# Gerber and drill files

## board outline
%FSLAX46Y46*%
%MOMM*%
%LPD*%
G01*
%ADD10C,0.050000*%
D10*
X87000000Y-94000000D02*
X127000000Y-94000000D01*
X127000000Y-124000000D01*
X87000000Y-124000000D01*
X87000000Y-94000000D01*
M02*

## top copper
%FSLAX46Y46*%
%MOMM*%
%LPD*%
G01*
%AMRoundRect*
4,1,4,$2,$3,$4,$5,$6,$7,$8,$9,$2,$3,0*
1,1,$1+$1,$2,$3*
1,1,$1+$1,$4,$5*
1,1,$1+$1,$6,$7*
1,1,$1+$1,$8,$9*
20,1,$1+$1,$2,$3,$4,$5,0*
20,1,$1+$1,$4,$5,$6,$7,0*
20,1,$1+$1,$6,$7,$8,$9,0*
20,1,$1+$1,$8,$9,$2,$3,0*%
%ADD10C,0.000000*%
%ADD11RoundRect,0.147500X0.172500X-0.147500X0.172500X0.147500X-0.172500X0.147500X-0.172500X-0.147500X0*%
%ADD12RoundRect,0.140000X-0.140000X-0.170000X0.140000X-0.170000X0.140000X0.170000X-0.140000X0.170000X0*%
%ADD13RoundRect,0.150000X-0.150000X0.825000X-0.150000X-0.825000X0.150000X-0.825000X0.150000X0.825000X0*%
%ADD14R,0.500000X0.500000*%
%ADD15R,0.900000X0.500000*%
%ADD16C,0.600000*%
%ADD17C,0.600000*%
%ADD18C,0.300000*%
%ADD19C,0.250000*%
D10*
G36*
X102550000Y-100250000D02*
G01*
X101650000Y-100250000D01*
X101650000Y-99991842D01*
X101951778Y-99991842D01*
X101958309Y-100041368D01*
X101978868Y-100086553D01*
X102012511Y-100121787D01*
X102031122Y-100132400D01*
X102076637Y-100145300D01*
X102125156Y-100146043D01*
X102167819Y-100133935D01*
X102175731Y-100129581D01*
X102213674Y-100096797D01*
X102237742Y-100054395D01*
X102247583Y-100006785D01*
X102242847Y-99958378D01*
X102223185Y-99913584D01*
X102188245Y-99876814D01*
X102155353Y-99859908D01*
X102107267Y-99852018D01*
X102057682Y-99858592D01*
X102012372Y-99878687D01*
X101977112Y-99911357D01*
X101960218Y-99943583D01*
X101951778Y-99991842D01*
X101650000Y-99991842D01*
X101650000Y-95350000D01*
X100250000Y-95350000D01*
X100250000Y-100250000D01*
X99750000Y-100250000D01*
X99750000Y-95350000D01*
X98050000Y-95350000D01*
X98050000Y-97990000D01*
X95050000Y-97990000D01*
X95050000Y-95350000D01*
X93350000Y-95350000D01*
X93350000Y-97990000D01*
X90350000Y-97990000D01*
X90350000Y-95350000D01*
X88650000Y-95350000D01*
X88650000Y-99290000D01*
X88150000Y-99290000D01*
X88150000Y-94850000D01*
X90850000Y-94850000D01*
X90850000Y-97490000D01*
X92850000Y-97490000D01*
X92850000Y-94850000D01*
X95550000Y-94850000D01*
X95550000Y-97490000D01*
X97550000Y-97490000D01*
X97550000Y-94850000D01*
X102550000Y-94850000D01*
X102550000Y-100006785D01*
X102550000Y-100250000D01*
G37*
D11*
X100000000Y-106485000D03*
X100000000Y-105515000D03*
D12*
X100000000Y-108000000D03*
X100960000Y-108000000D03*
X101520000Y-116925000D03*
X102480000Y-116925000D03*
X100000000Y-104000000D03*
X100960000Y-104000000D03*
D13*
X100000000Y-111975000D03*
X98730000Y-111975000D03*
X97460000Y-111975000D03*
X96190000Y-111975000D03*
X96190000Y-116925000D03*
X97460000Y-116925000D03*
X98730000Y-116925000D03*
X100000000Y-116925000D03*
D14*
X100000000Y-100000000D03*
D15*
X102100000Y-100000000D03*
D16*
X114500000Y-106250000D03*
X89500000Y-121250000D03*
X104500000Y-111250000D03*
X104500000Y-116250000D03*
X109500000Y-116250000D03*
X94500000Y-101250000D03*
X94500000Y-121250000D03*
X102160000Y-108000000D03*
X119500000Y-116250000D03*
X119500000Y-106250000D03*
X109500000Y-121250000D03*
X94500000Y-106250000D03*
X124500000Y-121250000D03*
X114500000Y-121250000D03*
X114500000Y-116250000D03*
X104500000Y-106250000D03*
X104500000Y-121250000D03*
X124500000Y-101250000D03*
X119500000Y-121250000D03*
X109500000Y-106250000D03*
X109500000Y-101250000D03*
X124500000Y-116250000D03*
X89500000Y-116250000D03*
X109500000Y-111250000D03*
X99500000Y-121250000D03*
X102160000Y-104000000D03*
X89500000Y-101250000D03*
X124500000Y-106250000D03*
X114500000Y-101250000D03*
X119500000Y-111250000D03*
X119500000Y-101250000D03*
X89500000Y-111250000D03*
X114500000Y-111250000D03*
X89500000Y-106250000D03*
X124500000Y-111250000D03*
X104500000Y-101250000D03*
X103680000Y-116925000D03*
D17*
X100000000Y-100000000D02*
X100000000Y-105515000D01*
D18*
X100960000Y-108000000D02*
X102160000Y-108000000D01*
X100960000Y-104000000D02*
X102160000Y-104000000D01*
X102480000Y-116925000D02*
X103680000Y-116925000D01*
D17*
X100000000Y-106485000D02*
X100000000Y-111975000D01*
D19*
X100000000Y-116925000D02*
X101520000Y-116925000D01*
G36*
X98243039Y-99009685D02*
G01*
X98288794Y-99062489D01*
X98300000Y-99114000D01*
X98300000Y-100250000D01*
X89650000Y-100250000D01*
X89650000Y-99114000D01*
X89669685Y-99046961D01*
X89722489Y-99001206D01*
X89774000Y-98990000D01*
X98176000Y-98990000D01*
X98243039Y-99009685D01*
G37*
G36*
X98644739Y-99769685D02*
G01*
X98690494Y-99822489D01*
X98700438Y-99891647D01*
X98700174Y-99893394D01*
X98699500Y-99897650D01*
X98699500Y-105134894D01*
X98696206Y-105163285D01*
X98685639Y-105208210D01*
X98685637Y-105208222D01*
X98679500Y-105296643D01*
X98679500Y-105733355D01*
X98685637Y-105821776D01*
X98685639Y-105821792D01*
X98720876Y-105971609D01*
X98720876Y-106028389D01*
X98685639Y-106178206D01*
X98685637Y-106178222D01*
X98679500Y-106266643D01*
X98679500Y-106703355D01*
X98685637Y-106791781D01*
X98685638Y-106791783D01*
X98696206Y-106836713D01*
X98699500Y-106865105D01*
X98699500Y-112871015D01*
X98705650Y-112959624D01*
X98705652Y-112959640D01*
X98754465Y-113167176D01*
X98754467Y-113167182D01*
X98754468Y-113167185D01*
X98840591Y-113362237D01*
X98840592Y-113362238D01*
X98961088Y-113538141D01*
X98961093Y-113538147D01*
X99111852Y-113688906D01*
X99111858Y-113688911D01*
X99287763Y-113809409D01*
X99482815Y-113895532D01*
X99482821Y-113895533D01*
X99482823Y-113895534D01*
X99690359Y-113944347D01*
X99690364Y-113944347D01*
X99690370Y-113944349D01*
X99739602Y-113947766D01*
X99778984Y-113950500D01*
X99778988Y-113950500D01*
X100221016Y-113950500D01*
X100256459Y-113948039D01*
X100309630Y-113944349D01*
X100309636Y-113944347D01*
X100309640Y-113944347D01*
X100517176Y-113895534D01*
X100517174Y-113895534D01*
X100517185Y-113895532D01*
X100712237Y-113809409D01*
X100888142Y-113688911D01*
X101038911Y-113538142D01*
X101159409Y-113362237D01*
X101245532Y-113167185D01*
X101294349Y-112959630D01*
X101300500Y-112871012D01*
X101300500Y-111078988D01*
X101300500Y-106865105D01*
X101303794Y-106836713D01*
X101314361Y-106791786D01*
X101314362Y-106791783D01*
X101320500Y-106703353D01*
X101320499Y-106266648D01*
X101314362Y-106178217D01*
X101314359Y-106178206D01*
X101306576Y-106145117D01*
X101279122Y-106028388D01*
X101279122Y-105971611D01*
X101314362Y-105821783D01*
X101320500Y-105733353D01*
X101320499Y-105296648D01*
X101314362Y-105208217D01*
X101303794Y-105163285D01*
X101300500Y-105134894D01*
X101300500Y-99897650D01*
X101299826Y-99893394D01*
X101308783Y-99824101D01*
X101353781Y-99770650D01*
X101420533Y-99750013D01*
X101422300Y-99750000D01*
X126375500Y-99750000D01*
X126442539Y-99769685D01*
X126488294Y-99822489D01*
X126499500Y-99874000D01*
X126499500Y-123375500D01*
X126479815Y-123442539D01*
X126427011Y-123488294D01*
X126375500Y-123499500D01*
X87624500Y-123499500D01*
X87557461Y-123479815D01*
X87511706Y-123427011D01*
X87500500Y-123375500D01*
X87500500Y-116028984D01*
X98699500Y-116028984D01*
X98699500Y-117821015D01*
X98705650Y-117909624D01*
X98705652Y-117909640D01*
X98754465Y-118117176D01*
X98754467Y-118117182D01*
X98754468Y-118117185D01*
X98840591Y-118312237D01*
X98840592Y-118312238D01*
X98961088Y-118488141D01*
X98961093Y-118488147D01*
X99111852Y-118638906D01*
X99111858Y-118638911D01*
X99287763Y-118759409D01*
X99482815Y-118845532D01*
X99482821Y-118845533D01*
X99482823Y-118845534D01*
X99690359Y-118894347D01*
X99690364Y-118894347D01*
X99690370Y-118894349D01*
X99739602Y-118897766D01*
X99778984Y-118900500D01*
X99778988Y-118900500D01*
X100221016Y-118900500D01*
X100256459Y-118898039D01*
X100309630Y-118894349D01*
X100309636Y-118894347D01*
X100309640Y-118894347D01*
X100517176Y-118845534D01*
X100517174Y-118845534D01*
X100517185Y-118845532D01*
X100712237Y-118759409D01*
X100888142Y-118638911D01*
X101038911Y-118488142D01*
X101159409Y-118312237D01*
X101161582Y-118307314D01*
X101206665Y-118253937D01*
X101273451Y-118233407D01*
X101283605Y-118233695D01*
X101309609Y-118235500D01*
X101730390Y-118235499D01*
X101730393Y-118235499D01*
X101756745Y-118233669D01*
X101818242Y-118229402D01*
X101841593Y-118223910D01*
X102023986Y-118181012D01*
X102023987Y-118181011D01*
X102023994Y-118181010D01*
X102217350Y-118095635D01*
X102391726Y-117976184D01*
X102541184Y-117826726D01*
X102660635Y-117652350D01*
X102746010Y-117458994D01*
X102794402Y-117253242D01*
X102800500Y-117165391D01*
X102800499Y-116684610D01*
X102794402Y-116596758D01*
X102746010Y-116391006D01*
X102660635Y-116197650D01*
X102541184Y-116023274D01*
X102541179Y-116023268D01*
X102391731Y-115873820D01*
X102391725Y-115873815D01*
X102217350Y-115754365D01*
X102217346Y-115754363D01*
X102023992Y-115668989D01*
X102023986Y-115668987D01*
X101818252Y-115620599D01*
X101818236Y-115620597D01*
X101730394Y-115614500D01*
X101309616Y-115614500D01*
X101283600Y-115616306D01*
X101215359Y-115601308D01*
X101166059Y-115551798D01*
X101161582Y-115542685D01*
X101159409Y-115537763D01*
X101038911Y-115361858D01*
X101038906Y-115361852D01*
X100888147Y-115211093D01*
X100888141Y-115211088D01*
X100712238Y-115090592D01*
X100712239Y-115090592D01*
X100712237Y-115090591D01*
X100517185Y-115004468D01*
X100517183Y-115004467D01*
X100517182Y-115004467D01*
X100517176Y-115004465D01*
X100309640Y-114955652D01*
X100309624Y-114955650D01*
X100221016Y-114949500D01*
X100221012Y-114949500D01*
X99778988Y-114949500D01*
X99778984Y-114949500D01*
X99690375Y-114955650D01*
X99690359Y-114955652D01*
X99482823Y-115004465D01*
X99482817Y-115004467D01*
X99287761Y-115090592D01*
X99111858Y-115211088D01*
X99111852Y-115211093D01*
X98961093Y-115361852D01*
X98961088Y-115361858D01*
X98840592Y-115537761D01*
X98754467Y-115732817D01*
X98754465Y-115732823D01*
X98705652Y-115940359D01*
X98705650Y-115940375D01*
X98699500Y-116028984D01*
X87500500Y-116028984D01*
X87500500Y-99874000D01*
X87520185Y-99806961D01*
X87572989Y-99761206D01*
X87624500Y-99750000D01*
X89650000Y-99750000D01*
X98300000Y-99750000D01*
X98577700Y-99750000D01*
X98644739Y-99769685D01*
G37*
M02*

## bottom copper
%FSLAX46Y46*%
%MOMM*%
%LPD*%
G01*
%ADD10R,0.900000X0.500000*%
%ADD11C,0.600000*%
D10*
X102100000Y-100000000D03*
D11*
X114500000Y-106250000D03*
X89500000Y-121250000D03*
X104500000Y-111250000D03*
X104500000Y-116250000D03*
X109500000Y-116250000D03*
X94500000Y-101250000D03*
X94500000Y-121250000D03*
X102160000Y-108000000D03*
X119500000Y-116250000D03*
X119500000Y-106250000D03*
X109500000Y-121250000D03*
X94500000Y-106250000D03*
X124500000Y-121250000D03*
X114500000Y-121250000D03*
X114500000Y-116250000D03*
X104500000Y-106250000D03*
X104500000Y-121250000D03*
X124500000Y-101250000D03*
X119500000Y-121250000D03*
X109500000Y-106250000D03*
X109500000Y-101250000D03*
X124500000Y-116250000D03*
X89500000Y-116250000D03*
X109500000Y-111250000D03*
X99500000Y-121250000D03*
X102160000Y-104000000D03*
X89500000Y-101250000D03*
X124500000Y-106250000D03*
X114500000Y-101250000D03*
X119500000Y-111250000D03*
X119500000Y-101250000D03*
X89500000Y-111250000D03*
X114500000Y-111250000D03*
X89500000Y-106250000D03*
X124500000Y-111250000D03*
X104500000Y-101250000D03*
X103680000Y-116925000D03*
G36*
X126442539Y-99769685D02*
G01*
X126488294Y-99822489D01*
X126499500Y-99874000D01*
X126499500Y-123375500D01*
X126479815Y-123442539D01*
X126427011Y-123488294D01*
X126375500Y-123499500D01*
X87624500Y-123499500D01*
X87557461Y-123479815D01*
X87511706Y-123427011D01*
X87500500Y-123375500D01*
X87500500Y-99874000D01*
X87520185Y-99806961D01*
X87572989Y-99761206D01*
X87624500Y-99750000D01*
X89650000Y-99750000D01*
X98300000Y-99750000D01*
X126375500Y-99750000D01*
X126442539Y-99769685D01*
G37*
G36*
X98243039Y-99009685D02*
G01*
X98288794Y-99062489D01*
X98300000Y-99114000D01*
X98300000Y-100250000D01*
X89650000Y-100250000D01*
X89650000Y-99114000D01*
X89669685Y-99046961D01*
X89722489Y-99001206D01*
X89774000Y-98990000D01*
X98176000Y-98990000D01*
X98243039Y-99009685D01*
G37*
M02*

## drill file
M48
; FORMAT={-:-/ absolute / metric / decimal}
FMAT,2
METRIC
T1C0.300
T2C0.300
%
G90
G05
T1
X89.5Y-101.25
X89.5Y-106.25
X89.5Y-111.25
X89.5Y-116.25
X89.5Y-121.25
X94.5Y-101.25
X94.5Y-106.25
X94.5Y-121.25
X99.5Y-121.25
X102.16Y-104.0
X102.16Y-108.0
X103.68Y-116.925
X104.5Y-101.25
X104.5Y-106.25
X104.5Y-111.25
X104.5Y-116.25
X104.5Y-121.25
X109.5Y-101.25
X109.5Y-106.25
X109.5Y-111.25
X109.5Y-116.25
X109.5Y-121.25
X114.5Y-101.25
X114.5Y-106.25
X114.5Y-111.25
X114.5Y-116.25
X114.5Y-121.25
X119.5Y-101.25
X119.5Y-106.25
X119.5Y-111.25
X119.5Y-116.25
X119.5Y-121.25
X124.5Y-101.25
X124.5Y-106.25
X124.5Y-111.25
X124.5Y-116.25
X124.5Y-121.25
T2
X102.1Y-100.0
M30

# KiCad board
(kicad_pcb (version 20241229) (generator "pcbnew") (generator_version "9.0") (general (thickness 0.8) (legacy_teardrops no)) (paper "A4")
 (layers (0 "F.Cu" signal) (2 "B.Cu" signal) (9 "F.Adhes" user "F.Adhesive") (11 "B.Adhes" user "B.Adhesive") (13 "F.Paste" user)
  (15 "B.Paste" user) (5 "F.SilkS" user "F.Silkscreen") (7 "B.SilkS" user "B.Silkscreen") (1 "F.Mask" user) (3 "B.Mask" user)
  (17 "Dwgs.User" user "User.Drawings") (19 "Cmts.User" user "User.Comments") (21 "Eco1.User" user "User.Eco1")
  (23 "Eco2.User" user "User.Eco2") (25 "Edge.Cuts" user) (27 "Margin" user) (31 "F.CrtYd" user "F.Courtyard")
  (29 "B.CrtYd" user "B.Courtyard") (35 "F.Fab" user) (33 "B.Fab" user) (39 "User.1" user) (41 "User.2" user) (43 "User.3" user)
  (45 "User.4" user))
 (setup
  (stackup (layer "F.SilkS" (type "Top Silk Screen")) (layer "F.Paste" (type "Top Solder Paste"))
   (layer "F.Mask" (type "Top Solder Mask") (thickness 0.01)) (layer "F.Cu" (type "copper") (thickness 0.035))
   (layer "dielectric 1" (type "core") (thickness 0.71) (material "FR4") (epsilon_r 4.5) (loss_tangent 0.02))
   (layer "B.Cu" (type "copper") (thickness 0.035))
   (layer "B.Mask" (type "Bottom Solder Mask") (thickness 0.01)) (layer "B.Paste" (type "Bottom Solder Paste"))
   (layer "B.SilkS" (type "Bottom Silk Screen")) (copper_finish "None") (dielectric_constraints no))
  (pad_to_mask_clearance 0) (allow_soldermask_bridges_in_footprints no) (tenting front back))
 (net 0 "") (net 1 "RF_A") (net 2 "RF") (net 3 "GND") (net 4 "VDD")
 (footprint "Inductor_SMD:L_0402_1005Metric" (layer "F.Cu") (at 100 106 90)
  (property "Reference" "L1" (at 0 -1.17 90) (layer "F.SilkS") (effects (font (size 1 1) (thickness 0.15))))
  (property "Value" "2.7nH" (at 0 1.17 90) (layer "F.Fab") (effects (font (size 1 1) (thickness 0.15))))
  (pad "1" smd roundrect (at -0.485 0 90) (size 0.59 0.64) (layers "F.Cu" "F.Mask" "F.Paste") (roundrect_rratio 0.25) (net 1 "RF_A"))
  (pad "2" smd roundrect (at 0.485 0 90) (size 0.59 0.64) (layers "F.Cu" "F.Mask" "F.Paste") (roundrect_rratio 0.25) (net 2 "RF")))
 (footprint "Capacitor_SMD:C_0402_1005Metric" (layer "F.Cu") (at 100.48 108)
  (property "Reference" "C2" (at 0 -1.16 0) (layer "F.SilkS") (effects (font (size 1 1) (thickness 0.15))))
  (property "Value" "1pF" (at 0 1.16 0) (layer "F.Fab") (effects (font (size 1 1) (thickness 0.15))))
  (pad "1" smd roundrect (at -0.48 0) (size 0.56 0.62) (layers "F.Cu" "F.Mask" "F.Paste") (roundrect_rratio 0.25) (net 1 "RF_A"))
  (pad "2" smd roundrect (at 0.48 0) (size 0.56 0.62) (layers "F.Cu" "F.Mask" "F.Paste") (roundrect_rratio 0.25) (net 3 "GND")))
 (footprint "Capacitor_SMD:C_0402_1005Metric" (layer "F.Cu") (at 102 116.925)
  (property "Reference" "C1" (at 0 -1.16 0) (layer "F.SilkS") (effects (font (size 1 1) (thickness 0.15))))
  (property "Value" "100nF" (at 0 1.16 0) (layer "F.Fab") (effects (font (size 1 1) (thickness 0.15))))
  (pad "1" smd roundrect (at -0.48 0) (size 0.56 0.62) (layers "F.Cu" "F.Mask" "F.Paste") (roundrect_rratio 0.25) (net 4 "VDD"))
  (pad "2" smd roundrect (at 0.48 0) (size 0.56 0.62) (layers "F.Cu" "F.Mask" "F.Paste") (roundrect_rratio 0.25) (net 3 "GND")))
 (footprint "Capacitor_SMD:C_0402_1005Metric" (layer "F.Cu") (at 100.48 104)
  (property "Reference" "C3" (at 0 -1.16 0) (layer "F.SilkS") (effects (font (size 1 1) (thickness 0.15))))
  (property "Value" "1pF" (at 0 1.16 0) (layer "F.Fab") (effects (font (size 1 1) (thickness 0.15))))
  (pad "1" smd roundrect (at -0.48 0) (size 0.56 0.62) (layers "F.Cu" "F.Mask" "F.Paste") (roundrect_rratio 0.25) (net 2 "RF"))
  (pad "2" smd roundrect (at 0.48 0) (size 0.56 0.62) (layers "F.Cu" "F.Mask" "F.Paste") (roundrect_rratio 0.25) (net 3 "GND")))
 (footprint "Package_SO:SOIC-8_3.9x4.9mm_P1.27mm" (layer "F.Cu") (at 98.095 114.45 -90)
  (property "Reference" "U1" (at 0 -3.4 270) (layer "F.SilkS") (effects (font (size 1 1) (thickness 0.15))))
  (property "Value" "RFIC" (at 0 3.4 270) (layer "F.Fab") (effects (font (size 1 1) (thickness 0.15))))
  (pad "1" smd roundrect (at -2.475 -1.905 270) (size 1.95 0.6) (layers "F.Cu" "F.Mask" "F.Paste") (roundrect_rratio 0.25) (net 1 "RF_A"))
  (pad "2" smd roundrect (at -2.475 -0.635 270) (size 1.95 0.6) (layers "F.Cu" "F.Mask" "F.Paste") (roundrect_rratio 0.25) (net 3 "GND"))
  (pad "3" smd roundrect (at -2.475 0.635 270) (size 1.95 0.6) (layers "F.Cu" "F.Mask" "F.Paste") (roundrect_rratio 0.25) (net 3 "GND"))
  (pad "4" smd roundrect (at -2.475 1.905 270) (size 1.95 0.6) (layers "F.Cu" "F.Mask" "F.Paste") (roundrect_rratio 0.25) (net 3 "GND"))
  (pad "5" smd roundrect (at 2.475 1.905 270) (size 1.95 0.6) (layers "F.Cu" "F.Mask" "F.Paste") (roundrect_rratio 0.25) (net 3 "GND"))
  (pad "6" smd roundrect (at 2.475 0.635 270) (size 1.95 0.6) (layers "F.Cu" "F.Mask" "F.Paste") (roundrect_rratio 0.25) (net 3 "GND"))
  (pad "7" smd roundrect (at 2.475 -0.635 270) (size 1.95 0.6) (layers "F.Cu" "F.Mask" "F.Paste") (roundrect_rratio 0.25) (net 3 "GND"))
  (pad "8" smd roundrect (at 2.475 -1.905 270) (size 1.95 0.6) (layers "F.Cu" "F.Mask" "F.Paste") (roundrect_rratio 0.25) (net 4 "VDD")))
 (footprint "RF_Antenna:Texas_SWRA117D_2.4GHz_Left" (layer "F.Cu") (at 100 100)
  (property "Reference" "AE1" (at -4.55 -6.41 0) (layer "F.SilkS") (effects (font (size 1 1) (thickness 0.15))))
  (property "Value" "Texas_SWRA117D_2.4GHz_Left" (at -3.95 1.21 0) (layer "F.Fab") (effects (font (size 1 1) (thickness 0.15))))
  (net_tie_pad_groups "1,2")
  (fp_poly
   (pts (xy -2.45 -2.51) (xy -4.45 -2.51) (xy -4.45 -5.15) (xy -7.15 -5.15) (xy -7.15 -2.51) (xy -9.15 -2.51) (xy -9.15 -5.15)
    (xy -11.85 -5.15) (xy -11.85 -0.71) (xy -11.35 -0.71) (xy -11.35 -4.65) (xy -9.65 -4.65) (xy -9.65 -2.01) (xy -6.65 -2.01)
    (xy -6.65 -4.65) (xy -4.95 -4.65) (xy -4.95 -2.01) (xy -1.95 -2.01) (xy -1.95 -4.65) (xy -0.25 -4.65) (xy -0.25 0.25) (xy 0.25 0.25)
    (xy 0.25 -4.65) (xy 1.65 -4.65) (xy 1.65 0.25) (xy 2.55 0.25) (xy 2.55 0.006785) (xy 2.247583 0.006785) (xy 2.237742 0.054395)
    (xy 2.213674 0.096797) (xy 2.175731 0.129581) (xy 2.167819 0.133935) (xy 2.125156 0.146043) (xy 2.076637 0.1453) (xy 2.031122 0.1324)
    (xy 2.012511 0.121787) (xy 1.978868 0.086553) (xy 1.958309 0.041368) (xy 1.951778 -0.008158) (xy 1.960218 -0.056417)
    (xy 1.977112 -0.088643) (xy 2.012372 -0.121313) (xy 2.057682 -0.141408) (xy 2.107267 -0.147982) (xy 2.155353 -0.140092)
    (xy 2.188245 -0.123186) (xy 2.223185 -0.086416) (xy 2.242847 -0.041622) (xy 2.247583 0.006785) (xy 2.55 0.006785) (xy 2.55 -5.15)
    (xy -2.45 -5.15) (xy -2.45 -2.51))
   (stroke (width 0) (type solid)) (fill yes) (layer "F.Cu"))
  (pad "1" connect rect (at 0 0) (size 0.5 0.5) (layers "F.Cu") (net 2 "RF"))
  (pad "2" thru_hole rect (at 2.1 0) (size 0.9 0.5) (drill 0.3) (layers "*.Cu") (remove_unused_layers no) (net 3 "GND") (zone_connect 2)))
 (gr_rect (start 87 94) (end 127 124) (stroke (width 0.05) (type default)) (fill no) (layer "Edge.Cuts"))
 (segment (start 100 100) (end 100 105.515) (width 0.6) (layer "F.Cu") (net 2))
 (segment (start 100.96 108) (end 102.16 108) (width 0.3) (layer "F.Cu") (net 3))
 (segment (start 100.96 104) (end 102.16 104) (width 0.3) (layer "F.Cu") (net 3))
 (segment (start 102.48 116.925) (end 103.68 116.925) (width 0.3) (layer "F.Cu") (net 3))
 (via (at 114.5 106.25) (size 0.6) (drill 0.3) (layers "F.Cu" "B.Cu") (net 3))
 (via (at 89.5 121.25) (size 0.6) (drill 0.3) (layers "F.Cu" "B.Cu") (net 3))
 (via (at 104.5 111.25) (size 0.6) (drill 0.3) (layers "F.Cu" "B.Cu") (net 3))
 (via (at 104.5 116.25) (size 0.6) (drill 0.3) (layers "F.Cu" "B.Cu") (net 3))
 (via (at 109.5 116.25) (size 0.6) (drill 0.3) (layers "F.Cu" "B.Cu") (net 3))
 (via (at 94.5 101.25) (size 0.6) (drill 0.3) (layers "F.Cu" "B.Cu") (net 3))
 (via (at 94.5 121.25) (size 0.6) (drill 0.3) (layers "F.Cu" "B.Cu") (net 3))
 (via (at 102.16 108) (size 0.6) (drill 0.3) (layers "F.Cu" "B.Cu") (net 3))
 (via (at 119.5 116.25) (size 0.6) (drill 0.3) (layers "F.Cu" "B.Cu") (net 3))
 (via (at 119.5 106.25) (size 0.6) (drill 0.3) (layers "F.Cu" "B.Cu") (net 3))
 (via (at 109.5 121.25) (size 0.6) (drill 0.3) (layers "F.Cu" "B.Cu") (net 3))
 (via (at 94.5 106.25) (size 0.6) (drill 0.3) (layers "F.Cu" "B.Cu") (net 3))
 (via (at 124.5 121.25) (size 0.6) (drill 0.3) (layers "F.Cu" "B.Cu") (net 3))
 (via (at 114.5 121.25) (size 0.6) (drill 0.3) (layers "F.Cu" "B.Cu") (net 3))
 (via (at 114.5 116.25) (size 0.6) (drill 0.3) (layers "F.Cu" "B.Cu") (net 3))
 (via (at 104.5 106.25) (size 0.6) (drill 0.3) (layers "F.Cu" "B.Cu") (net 3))
 (via (at 104.5 121.25) (size 0.6) (drill 0.3) (layers "F.Cu" "B.Cu") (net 3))
 (via (at 124.5 101.25) (size 0.6) (drill 0.3) (layers "F.Cu" "B.Cu") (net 3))
 (via (at 119.5 121.25) (size 0.6) (drill 0.3) (layers "F.Cu" "B.Cu") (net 3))
 (via (at 109.5 106.25) (size 0.6) (drill 0.3) (layers "F.Cu" "B.Cu") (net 3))
 (via (at 109.5 101.25) (size 0.6) (drill 0.3) (layers "F.Cu" "B.Cu") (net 3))
 (via (at 124.5 116.25) (size 0.6) (drill 0.3) (layers "F.Cu" "B.Cu") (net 3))
 (via (at 89.5 116.25) (size 0.6) (drill 0.3) (layers "F.Cu" "B.Cu") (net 3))
 (via (at 109.5 111.25) (size 0.6) (drill 0.3) (layers "F.Cu" "B.Cu") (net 3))
 (via (at 99.5 121.25) (size 0.6) (drill 0.3) (layers "F.Cu" "B.Cu") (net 3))
 (via (at 102.16 104) (size 0.6) (drill 0.3) (layers "F.Cu" "B.Cu") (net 3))
 (via (at 89.5 101.25) (size 0.6) (drill 0.3) (layers "F.Cu" "B.Cu") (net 3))
 (via (at 124.5 106.25) (size 0.6) (drill 0.3) (layers "F.Cu" "B.Cu") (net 3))
 (via (at 114.5 101.25) (size 0.6) (drill 0.3) (layers "F.Cu" "B.Cu") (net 3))
 (via (at 119.5 111.25) (size 0.6) (drill 0.3) (layers "F.Cu" "B.Cu") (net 3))
 (via (at 119.5 101.25) (size 0.6) (drill 0.3) (layers "F.Cu" "B.Cu") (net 3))
 (via (at 89.5 111.25) (size 0.6) (drill 0.3) (layers "F.Cu" "B.Cu") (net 3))
 (via (at 114.5 111.25) (size 0.6) (drill 0.3) (layers "F.Cu" "B.Cu") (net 3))
 (via (at 89.5 106.25) (size 0.6) (drill 0.3) (layers "F.Cu" "B.Cu") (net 3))
 (via (at 124.5 111.25) (size 0.6) (drill 0.3) (layers "F.Cu" "B.Cu") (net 3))
 (via (at 104.5 101.25) (size 0.6) (drill 0.3) (layers "F.Cu" "B.Cu") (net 3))
 (via (at 103.68 116.925) (size 0.6) (drill 0.3) (layers "F.Cu" "B.Cu") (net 3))
 (segment (start 100 106.485) (end 100 111.975) (width 0.6) (layer "F.Cu") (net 1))
 (segment (start 100 116.925) (end 101.52 116.925) (width 0.25) (layer "F.Cu") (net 4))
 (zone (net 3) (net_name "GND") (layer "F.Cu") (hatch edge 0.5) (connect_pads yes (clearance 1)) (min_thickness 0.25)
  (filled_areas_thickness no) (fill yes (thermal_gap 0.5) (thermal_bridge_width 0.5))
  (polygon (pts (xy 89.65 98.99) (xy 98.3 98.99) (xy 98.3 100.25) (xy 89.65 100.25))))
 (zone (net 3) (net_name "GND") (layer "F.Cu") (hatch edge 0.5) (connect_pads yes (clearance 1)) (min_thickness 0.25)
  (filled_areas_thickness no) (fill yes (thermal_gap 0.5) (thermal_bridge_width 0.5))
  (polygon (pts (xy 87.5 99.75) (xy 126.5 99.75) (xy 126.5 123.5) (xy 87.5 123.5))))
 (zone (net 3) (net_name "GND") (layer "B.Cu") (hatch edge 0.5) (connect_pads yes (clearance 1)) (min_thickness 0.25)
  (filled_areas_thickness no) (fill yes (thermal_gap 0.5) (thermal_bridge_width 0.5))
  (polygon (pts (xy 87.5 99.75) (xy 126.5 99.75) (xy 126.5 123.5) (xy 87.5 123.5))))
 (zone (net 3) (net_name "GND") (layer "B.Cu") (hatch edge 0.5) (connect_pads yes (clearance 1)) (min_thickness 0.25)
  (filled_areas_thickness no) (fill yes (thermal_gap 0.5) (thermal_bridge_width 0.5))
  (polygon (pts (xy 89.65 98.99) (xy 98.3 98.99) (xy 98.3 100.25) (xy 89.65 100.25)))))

